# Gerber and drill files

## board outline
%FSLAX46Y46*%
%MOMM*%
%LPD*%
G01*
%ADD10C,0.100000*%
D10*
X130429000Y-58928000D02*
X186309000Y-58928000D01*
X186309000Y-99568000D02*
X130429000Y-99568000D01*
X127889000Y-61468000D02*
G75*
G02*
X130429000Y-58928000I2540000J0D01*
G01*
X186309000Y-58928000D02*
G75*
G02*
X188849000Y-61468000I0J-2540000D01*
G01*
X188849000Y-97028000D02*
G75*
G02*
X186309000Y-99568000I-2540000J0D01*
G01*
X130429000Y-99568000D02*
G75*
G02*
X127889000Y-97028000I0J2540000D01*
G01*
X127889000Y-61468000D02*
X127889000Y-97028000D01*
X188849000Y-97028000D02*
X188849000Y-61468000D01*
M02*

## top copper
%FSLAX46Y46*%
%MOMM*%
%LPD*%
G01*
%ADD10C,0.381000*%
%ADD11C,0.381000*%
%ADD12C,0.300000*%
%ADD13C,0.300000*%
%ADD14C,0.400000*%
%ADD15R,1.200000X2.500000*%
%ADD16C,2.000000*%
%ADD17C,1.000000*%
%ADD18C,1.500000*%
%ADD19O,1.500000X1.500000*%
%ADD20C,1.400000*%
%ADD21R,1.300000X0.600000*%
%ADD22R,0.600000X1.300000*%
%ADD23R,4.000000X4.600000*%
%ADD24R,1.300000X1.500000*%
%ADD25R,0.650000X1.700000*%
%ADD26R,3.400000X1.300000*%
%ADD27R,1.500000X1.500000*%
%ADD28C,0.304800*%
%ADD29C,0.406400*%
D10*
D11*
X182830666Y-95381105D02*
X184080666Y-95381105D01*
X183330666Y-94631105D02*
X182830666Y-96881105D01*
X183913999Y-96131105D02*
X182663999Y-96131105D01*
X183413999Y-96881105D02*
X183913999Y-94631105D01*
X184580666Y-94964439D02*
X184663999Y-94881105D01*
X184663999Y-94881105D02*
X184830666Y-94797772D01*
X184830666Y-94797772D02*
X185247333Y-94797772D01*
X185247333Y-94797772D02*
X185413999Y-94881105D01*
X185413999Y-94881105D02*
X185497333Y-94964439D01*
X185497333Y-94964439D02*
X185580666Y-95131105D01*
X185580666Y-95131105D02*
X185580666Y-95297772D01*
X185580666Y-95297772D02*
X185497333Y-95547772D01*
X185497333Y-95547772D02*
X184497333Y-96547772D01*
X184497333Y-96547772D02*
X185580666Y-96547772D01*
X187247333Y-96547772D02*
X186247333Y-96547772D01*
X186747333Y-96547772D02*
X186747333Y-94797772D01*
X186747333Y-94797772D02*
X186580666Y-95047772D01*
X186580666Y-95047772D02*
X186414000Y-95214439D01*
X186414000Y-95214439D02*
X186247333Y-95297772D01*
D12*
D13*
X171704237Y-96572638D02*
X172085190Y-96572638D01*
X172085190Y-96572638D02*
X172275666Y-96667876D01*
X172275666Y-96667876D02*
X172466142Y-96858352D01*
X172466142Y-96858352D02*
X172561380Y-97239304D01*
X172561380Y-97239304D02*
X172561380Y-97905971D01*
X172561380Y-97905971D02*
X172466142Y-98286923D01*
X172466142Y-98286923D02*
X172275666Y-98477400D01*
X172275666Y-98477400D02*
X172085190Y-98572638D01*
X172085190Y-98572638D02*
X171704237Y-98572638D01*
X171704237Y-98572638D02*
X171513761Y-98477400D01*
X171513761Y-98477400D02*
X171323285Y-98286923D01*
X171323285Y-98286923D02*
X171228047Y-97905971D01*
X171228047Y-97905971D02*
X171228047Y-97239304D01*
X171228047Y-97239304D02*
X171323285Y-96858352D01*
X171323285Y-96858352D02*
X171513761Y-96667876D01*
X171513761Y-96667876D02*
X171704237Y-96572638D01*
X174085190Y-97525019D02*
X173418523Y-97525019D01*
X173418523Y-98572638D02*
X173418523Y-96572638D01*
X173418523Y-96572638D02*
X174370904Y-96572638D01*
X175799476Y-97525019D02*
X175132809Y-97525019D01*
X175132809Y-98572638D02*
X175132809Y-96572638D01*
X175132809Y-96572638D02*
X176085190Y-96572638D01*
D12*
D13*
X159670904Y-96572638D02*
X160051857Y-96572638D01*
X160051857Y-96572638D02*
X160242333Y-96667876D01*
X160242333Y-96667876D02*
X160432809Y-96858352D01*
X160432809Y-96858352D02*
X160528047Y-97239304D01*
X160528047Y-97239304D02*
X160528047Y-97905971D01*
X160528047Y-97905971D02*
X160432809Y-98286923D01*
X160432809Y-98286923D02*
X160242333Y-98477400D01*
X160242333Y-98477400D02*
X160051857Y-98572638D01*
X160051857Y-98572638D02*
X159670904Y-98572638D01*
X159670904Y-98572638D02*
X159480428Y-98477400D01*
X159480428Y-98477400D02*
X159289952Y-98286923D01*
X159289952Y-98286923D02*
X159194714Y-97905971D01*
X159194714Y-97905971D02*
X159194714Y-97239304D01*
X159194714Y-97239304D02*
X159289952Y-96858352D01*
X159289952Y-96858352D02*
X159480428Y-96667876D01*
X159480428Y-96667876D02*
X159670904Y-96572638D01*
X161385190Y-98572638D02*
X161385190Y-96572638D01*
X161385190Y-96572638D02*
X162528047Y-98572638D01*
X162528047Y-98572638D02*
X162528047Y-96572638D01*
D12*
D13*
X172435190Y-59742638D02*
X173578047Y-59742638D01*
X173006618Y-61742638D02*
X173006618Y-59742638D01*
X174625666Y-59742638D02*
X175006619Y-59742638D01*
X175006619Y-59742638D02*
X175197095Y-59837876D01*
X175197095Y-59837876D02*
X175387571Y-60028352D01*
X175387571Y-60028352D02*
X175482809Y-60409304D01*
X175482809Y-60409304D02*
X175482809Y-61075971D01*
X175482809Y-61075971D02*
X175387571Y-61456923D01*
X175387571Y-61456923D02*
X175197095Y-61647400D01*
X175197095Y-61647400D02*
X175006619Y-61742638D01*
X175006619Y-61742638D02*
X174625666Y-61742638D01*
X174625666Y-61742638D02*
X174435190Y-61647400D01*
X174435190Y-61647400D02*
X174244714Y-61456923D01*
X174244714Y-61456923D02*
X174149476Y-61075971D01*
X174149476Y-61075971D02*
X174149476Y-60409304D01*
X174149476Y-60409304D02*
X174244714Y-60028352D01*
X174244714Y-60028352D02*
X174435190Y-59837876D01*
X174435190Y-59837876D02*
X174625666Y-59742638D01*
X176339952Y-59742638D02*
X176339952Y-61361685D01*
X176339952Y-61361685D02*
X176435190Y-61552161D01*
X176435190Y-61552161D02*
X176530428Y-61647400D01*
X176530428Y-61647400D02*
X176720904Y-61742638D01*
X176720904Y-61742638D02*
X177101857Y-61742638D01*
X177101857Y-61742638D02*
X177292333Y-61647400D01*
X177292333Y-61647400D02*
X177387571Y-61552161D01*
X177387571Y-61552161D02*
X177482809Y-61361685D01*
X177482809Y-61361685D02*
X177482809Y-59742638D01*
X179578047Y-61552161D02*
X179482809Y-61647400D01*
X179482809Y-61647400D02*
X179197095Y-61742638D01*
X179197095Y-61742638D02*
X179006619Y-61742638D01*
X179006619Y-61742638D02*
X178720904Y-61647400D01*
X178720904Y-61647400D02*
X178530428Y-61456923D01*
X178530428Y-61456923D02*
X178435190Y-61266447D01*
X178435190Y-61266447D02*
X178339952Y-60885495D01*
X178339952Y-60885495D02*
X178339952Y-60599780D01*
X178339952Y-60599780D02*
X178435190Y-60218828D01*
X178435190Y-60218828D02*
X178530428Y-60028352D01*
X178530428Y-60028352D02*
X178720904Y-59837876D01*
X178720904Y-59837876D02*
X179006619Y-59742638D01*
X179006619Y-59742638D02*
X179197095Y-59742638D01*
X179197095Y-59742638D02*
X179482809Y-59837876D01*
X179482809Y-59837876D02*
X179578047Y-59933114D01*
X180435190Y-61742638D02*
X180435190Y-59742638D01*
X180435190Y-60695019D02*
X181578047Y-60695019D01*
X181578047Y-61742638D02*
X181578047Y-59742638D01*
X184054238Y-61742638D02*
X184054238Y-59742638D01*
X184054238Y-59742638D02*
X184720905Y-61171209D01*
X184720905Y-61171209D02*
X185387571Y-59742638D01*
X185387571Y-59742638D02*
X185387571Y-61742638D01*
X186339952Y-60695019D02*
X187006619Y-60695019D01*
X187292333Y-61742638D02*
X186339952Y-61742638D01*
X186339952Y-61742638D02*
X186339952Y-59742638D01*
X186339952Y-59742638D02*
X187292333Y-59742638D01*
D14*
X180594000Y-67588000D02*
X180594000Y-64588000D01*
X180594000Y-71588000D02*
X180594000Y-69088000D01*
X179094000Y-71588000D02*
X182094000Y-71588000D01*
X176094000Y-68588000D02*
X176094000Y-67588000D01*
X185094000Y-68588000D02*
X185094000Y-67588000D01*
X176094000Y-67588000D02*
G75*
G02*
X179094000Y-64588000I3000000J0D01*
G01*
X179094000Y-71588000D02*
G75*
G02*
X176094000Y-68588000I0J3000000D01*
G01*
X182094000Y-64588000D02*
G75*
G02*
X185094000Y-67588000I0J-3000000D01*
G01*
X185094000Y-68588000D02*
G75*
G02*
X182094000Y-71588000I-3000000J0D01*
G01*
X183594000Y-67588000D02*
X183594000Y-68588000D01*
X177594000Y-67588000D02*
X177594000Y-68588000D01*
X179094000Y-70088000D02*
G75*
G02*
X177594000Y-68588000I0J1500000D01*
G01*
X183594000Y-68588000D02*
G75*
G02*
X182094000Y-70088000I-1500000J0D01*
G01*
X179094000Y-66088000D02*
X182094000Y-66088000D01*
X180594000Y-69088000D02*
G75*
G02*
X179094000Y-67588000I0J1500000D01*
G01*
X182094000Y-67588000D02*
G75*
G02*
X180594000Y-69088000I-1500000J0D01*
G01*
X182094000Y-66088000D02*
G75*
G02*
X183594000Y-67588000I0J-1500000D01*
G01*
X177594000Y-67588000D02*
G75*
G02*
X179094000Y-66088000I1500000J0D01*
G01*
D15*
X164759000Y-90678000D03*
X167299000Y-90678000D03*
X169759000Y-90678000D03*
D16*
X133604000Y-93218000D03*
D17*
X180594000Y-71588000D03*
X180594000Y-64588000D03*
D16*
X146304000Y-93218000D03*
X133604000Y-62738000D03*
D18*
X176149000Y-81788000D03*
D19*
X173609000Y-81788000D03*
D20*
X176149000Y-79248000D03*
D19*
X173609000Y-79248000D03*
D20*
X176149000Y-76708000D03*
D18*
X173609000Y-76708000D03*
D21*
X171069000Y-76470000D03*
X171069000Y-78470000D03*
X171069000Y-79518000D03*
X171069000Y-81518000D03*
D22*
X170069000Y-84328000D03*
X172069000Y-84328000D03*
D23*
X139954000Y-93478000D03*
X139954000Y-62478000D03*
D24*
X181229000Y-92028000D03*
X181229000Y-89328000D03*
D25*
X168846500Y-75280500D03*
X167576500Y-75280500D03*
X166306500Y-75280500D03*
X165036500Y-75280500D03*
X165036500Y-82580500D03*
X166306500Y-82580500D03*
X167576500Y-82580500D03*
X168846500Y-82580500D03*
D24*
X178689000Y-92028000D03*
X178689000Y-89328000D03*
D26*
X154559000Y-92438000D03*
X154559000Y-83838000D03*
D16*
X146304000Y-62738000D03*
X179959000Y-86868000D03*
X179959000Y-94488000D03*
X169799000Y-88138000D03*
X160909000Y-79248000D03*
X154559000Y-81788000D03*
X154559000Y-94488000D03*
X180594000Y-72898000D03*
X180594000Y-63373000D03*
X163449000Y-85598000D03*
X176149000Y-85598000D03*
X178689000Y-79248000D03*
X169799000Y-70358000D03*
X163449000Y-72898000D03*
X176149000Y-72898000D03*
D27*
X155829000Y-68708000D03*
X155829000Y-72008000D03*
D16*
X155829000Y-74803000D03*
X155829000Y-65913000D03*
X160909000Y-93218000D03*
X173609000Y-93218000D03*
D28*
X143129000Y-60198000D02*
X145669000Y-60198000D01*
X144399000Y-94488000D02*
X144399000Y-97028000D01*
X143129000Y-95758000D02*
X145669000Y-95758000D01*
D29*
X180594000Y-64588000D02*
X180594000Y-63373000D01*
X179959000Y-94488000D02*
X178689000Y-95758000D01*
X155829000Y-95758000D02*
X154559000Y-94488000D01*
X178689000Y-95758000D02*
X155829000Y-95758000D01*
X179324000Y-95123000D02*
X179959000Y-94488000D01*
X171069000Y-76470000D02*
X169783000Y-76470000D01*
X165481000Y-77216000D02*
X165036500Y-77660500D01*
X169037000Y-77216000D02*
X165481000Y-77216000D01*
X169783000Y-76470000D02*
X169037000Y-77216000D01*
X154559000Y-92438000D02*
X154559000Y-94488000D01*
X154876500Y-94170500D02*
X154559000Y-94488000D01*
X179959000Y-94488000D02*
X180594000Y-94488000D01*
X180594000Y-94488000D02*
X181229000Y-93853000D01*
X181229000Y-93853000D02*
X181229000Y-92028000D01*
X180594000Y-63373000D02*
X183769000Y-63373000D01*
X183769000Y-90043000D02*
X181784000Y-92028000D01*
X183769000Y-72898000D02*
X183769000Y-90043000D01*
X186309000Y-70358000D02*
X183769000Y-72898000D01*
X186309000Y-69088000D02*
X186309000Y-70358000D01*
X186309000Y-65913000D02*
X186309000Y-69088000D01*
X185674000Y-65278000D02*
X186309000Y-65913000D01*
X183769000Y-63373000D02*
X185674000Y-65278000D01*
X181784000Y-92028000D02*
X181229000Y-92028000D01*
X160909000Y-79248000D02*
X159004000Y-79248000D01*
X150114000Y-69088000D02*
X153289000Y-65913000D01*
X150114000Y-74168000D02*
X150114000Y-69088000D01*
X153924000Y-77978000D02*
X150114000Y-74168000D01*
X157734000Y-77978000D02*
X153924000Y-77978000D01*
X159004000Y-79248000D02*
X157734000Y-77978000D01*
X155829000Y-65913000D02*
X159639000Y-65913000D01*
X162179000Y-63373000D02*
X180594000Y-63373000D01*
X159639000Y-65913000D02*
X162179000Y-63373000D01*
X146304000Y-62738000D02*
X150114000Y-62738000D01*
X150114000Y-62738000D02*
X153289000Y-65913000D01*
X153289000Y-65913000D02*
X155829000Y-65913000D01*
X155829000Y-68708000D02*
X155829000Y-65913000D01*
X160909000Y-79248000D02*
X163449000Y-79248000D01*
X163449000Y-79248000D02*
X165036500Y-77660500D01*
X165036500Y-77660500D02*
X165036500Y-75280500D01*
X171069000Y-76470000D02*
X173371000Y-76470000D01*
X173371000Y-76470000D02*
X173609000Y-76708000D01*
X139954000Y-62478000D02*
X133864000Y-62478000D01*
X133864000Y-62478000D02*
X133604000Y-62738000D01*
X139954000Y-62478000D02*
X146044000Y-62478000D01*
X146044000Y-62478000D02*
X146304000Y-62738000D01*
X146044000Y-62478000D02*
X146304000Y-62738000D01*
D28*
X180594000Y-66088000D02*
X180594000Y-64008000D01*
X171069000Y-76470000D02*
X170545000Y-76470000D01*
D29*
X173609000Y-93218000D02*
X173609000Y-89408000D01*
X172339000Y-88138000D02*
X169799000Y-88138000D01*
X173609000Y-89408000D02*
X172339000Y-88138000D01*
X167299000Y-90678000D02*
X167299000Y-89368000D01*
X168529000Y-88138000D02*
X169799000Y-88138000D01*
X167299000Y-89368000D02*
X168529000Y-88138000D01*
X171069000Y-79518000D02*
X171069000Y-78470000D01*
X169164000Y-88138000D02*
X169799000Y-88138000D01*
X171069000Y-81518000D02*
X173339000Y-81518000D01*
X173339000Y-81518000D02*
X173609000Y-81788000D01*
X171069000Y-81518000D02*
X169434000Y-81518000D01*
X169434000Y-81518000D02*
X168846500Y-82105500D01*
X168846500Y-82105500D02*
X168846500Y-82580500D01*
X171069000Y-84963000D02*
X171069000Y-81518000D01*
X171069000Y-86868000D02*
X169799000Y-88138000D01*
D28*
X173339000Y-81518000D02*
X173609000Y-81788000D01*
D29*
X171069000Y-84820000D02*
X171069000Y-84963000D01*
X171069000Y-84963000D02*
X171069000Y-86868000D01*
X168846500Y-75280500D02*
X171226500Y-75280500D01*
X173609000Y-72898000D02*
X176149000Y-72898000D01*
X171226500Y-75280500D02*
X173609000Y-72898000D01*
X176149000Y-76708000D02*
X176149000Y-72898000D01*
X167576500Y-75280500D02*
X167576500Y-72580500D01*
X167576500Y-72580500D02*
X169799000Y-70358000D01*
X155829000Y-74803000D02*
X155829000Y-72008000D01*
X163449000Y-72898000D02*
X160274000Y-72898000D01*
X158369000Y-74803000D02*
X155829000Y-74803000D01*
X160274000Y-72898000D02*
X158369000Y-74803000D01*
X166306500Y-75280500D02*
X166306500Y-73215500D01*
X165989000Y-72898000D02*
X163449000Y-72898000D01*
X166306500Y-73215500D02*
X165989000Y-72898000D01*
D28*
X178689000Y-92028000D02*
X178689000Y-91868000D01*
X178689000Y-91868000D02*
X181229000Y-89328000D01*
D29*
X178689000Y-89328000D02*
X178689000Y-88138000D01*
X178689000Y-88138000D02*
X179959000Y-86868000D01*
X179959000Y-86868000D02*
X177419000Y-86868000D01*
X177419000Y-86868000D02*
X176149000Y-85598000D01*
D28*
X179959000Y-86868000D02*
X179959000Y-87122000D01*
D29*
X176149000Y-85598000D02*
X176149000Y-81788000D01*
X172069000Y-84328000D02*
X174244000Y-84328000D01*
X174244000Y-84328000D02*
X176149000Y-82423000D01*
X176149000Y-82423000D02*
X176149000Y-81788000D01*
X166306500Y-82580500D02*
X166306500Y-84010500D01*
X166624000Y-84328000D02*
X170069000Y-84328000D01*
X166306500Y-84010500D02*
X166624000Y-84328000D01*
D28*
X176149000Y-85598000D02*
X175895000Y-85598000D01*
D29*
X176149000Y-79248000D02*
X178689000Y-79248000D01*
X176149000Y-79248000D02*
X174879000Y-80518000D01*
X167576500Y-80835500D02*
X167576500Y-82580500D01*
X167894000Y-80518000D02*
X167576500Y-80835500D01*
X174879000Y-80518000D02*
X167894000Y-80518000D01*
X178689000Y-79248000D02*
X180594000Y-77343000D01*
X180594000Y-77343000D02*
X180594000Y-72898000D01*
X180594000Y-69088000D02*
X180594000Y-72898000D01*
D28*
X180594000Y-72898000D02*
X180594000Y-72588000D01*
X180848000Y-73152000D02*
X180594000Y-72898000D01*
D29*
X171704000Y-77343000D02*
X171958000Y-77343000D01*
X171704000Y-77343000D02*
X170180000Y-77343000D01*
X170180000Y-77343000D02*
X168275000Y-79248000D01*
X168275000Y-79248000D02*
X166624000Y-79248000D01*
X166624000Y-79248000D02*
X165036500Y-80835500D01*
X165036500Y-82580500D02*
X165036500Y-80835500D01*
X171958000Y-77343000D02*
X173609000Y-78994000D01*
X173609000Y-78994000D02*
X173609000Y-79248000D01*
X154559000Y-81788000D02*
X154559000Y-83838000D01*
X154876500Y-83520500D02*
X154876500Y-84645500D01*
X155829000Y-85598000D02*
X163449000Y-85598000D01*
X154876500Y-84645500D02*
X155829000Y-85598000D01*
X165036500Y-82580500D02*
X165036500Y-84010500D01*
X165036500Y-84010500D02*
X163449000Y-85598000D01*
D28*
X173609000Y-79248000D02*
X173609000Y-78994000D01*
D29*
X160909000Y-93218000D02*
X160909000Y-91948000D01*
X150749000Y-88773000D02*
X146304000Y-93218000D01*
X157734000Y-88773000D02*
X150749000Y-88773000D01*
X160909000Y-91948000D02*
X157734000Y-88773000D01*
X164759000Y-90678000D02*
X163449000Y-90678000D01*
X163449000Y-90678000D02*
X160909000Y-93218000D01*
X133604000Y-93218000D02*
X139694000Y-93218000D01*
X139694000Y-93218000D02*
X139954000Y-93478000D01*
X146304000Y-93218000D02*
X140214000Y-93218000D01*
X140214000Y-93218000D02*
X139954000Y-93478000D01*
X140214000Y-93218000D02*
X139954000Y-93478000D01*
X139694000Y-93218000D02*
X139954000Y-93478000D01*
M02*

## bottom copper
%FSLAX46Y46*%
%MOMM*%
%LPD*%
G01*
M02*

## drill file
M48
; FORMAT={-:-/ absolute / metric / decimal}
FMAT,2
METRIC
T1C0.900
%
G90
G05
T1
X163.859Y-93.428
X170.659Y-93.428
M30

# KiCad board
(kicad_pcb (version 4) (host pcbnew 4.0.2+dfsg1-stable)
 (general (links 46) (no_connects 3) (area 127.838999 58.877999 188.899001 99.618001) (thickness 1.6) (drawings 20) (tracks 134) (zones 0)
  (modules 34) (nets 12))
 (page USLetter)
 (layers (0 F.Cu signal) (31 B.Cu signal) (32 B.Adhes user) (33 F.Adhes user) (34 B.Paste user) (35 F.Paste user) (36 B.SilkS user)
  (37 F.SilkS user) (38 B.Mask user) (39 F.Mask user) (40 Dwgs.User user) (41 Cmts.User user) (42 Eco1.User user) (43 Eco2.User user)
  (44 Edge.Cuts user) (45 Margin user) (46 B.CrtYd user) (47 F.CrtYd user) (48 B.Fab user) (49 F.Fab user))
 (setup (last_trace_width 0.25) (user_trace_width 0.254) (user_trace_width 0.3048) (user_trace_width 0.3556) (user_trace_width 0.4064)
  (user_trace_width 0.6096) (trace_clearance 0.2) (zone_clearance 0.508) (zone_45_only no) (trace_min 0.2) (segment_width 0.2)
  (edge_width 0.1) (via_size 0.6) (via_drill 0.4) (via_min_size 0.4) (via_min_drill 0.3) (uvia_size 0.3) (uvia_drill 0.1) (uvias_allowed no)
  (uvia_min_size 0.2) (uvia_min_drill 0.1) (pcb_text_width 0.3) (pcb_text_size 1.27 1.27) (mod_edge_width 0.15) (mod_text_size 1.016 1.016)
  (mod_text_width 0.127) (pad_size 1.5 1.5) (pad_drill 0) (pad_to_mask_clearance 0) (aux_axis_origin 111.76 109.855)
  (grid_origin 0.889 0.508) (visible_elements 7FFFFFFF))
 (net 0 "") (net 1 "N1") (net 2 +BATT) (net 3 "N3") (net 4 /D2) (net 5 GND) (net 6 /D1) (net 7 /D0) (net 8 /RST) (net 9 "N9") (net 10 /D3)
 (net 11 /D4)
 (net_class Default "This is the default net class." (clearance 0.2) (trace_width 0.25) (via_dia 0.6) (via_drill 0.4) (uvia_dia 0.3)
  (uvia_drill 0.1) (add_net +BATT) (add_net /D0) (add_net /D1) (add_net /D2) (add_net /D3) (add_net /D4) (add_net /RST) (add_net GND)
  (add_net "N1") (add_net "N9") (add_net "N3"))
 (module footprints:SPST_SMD (layer F.Cu) (at 167.259 90.678)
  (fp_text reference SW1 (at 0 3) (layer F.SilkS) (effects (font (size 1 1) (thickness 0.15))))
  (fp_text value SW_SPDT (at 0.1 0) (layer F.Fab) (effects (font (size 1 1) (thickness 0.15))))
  (pad "" np_thru_hole circle (at 3.4 2.75) (size 0.9 0.9) (drill 0.9) (layers *.Cu *.Mask))
  (pad 1 smd rect (at -2.5 0) (size 1.2 2.5) (layers F.Cu F.Paste F.Mask) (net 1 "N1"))
  (pad 2 smd rect (at 0.04 0) (size 1.2 2.5) (layers F.Cu F.Paste F.Mask) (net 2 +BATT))
  (pad 3 smd rect (at 2.5 0) (size 1.2 2.5) (layers F.Cu F.Paste F.Mask) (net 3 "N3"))
  (pad "" np_thru_hole circle (at -3.4 2.75) (size 0.9 0.9) (drill 0.9) (layers *.Cu *.Mask)))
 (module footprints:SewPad (layer F.Cu) (at 133.604 93.218)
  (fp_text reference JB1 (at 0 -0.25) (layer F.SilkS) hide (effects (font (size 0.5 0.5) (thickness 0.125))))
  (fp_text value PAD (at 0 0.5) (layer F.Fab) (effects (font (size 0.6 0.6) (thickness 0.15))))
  (pad 1 smd circle (at 0 0) (size 2 2) (layers F.Cu F.Mask) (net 1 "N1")))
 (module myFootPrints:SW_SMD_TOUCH (layer F.Cu) (at 180.594 69.088)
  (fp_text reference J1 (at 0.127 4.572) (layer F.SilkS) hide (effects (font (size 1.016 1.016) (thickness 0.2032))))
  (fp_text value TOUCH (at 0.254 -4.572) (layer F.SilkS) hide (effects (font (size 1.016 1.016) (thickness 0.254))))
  (fp_line (start 0 -1.5) (end 0 -4.5) (layer F.Cu) (width 0.4)) (fp_line (start 0 2.5) (end 0 0) (layer F.Cu) (width 0.4))
  (fp_line (start -1.5 2.5) (end 1.5 2.5) (layer F.Cu) (width 0.4))
  (fp_line (start -4.5 -0.5) (end -4.5 -1.5) (layer F.Cu) (width 0.4))
  (fp_line (start 4.5 -0.5) (end 4.5 -1.5) (layer F.Cu) (width 0.4))
  (fp_arc (start -1.5 -1.5) (end -4.5 -1.5) (angle 90) (layer F.Cu) (width 0.4))
  (fp_arc (start -1.5 -0.5) (end -1.5 2.5) (angle 90) (layer F.Cu) (width 0.4))
  (fp_arc (start 1.5 -1.5) (end 1.5 -4.5) (angle 90) (layer F.Cu) (width 0.4))
  (fp_arc (start 1.5 -0.5) (end 4.5 -0.5) (angle 90) (layer F.Cu) (width 0.4))
  (fp_line (start 3 -1.5) (end 3 -0.5) (layer F.Cu) (width 0.4))
  (fp_line (start -3 -1.5) (end -3 -0.5) (layer F.Cu) (width 0.4))
  (fp_arc (start -1.5 -0.5) (end -1.5 1) (angle 90) (layer F.Cu) (width 0.4))
  (fp_arc (start 1.5 -0.5) (end 3 -0.5) (angle 90) (layer F.Cu) (width 0.4))
  (fp_line (start -1.5 -3) (end 1.5 -3) (layer F.Cu) (width 0.4))
  (fp_arc (start 0 -1.5) (end 0 0) (angle 90) (layer F.Cu) (width 0.4))
  (fp_arc (start 0 -1.5) (end 1.5 -1.5) (angle 90) (layer F.Cu) (width 0.4))
  (fp_arc (start 1.5 -1.5) (end 1.5 -3) (angle 90) (layer F.Cu) (width 0.4))
  (fp_arc (start -1.5 -1.5) (end -3 -1.5) (angle 90) (layer F.Cu) (width 0.4))
  (pad 2 smd circle (at 0 2.5) (size 1 1) (layers F.Cu) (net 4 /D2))
  (pad 1 smd circle (at 0 -4.5) (size 1 1) (layers F.Cu) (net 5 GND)))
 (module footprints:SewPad (layer F.Cu) (at 146.304 93.218)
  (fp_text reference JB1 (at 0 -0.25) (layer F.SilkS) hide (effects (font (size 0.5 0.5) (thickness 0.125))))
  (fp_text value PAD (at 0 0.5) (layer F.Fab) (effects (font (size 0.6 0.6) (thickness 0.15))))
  (pad 1 smd circle (at 0 0) (size 2 2) (layers F.Cu F.Mask) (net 1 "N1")))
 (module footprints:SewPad (layer F.Cu) (at 133.604 62.738)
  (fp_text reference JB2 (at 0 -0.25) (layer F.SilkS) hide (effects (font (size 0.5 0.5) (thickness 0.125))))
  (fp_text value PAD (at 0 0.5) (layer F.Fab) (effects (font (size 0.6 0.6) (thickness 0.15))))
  (pad 1 smd circle (at 0 0) (size 2 2) (layers F.Cu F.Mask) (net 5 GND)))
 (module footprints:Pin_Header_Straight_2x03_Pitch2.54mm (layer F.Cu) (at 176.149 81.788 180)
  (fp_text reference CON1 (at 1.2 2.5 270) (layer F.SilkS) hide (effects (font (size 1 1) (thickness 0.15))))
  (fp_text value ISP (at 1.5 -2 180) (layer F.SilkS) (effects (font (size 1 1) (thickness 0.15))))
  (pad 1 smd circle (at 0 0 180) (size 1.5 1.5) (layers F.Cu) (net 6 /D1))
  (pad 2 smd oval (at 2.54 0 180) (size 1.5 1.5) (layers F.Cu) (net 2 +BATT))
  (pad 3 smd circle (at 0 2.54 180) (size 1.4 1.4) (layers F.Cu) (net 4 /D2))
  (pad 4 smd oval (at 2.54 2.54 180) (size 1.5 1.5) (layers F.Cu) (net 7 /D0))
  (pad 5 smd circle (at 0 5.08 180) (size 1.4 1.4) (layers F.Cu) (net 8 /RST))
  (pad 6 smd circle (at 2.54 5.08 180) (size 1.5 1.5) (layers F.Cu) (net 5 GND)))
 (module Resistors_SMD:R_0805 (layer F.Cu) (at 171.069 77.47 270)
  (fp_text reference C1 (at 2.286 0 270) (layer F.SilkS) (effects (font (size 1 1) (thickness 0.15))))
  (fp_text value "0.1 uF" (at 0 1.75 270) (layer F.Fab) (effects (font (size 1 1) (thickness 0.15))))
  (pad 1 smd rect (at -1 0 270) (size 0.6 1.3) (layers F.Cu F.Paste F.Mask) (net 5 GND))
  (pad 2 smd rect (at 1 0 270) (size 0.6 1.3) (layers F.Cu F.Paste F.Mask) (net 2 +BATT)))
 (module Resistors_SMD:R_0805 (layer F.Cu) (at 171.069 80.518 270)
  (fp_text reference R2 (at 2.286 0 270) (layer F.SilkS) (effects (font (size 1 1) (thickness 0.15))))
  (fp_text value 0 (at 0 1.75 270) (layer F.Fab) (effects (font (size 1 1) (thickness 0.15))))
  (pad 1 smd rect (at -1 0 270) (size 0.6 1.3) (layers F.Cu F.Paste F.Mask) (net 2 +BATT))
  (pad 2 smd rect (at 1 0 270) (size 0.6 1.3) (layers F.Cu F.Paste F.Mask) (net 2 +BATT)))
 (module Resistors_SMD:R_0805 (layer F.Cu) (at 171.069 84.328)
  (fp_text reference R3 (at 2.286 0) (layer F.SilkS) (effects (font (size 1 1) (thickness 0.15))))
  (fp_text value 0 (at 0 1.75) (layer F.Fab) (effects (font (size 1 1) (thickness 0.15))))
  (pad 1 smd rect (at -1 0) (size 0.6 1.3) (layers F.Cu F.Paste F.Mask) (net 6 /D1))
  (pad 2 smd rect (at 1 0) (size 0.6 1.3) (layers F.Cu F.Paste F.Mask) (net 6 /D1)))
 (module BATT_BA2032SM (layer F.Cu) (at 139.954 77.978 90)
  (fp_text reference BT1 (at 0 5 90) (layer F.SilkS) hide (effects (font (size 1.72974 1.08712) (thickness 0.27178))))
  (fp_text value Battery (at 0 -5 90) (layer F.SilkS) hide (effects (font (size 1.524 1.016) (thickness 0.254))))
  (pad 1 smd rect (at -15.5 0 90) (size 4.6 4) (layers F.Cu F.Paste F.Mask) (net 1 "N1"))
  (pad 2 smd rect (at 15.5 0 90) (size 4.6 4) (layers F.Cu F.Paste F.Mask) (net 5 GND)))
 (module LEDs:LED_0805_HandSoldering (layer F.Cu) (at 181.229 90.678 90)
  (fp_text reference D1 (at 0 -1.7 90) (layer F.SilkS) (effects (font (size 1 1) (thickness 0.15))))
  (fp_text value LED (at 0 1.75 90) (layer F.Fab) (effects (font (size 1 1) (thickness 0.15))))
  (pad 1 smd rect (at -1.35 0 90) (size 1.5 1.3) (layers F.Cu F.Paste F.Mask) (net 5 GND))
  (pad 2 smd rect (at 1.35 0 90) (size 1.5 1.3) (layers F.Cu F.Paste F.Mask) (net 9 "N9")))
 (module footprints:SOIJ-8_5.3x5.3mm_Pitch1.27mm (layer F.Cu) (at 166.9415 78.9305 270)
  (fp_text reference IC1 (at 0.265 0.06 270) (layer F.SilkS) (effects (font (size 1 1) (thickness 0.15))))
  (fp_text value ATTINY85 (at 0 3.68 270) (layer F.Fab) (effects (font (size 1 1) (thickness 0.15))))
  (pad 1 smd rect (at -3.65 -1.905 270) (size 1.7 0.65) (layers F.Cu F.Paste F.Mask) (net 8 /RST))
  (pad 2 smd rect (at -3.65 -0.635 270) (size 1.7 0.65) (layers F.Cu F.Paste F.Mask) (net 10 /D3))
  (pad 3 smd rect (at -3.65 0.635 270) (size 1.7 0.65) (layers F.Cu F.Paste F.Mask) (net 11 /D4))
  (pad 4 smd rect (at -3.65 1.905 270) (size 1.7 0.65) (layers F.Cu F.Paste F.Mask) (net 5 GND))
  (pad 5 smd rect (at 3.65 1.905 270) (size 1.7 0.65) (layers F.Cu F.Paste F.Mask) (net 7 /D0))
  (pad 6 smd rect (at 3.65 0.635 270) (size 1.7 0.65) (layers F.Cu F.Paste F.Mask) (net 6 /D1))
  (pad 7 smd rect (at 3.65 -0.635 270) (size 1.7 0.65) (layers F.Cu F.Paste F.Mask) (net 4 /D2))
  (pad 8 smd rect (at 3.65 -1.905 270) (size 1.7 0.65) (layers F.Cu F.Paste F.Mask) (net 2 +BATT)))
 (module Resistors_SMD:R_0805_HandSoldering (layer F.Cu) (at 178.689 90.678 90)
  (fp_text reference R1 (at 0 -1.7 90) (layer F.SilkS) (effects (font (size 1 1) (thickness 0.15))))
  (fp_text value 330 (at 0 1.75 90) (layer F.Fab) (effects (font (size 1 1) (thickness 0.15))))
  (pad 1 smd rect (at -1.35 0 90) (size 1.5 1.3) (layers F.Cu F.Paste F.Mask) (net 9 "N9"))
  (pad 2 smd rect (at 1.35 0 90) (size 1.5 1.3) (layers F.Cu F.Paste F.Mask) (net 6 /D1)))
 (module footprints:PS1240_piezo (layer F.Cu) (at 154.559 88.138 90)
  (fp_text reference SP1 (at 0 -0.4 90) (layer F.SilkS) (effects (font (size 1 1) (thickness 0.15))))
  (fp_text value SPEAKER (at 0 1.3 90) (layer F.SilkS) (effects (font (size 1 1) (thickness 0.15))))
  (pad 1 smd rect (at -4.3 0 90) (size 1.3 3.4) (layers F.Cu F.Paste F.Mask) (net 5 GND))
  (pad 2 smd rect (at 4.3 0 90) (size 1.3 3.4) (layers F.Cu F.Paste F.Mask) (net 7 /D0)))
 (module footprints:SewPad (layer F.Cu) (at 146.304 62.738)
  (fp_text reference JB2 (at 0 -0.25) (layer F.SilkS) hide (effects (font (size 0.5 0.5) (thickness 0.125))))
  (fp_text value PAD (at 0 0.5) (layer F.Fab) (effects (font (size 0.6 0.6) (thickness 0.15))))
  (pad 1 smd circle (at 0 0) (size 2 2) (layers F.Cu F.Mask) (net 5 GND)))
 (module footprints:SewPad (layer F.Cu) (at 179.959 86.868 90)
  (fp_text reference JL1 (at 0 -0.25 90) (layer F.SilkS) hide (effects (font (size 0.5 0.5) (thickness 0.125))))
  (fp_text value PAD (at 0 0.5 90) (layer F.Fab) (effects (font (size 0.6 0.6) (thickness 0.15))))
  (pad 1 smd circle (at 0 0 90) (size 2 2) (layers F.Cu F.Mask) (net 6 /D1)))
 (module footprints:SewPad (layer F.Cu) (at 179.959 94.488 90)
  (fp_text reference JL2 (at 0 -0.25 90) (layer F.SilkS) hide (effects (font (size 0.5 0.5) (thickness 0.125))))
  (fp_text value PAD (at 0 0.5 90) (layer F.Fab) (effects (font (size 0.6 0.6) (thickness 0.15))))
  (pad 1 smd circle (at 0 0 90) (size 2 2) (layers F.Cu F.Mask) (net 5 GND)))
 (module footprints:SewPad (layer F.Cu) (at 169.799 88.138)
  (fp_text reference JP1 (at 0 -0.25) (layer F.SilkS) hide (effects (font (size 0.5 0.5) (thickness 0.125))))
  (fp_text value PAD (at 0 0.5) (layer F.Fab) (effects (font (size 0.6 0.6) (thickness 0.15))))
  (pad 1 smd circle (at 0 0) (size 2 2) (layers F.Cu F.Mask) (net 2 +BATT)))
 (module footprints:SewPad (layer F.Cu) (at 160.909 79.248)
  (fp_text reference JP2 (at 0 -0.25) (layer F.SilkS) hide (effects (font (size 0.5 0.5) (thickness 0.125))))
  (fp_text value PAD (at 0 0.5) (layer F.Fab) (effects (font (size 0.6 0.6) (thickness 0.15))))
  (pad 1 smd circle (at 0 0) (size 2 2) (layers F.Cu F.Mask) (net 5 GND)))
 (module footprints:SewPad (layer F.Cu) (at 154.559 81.788 180)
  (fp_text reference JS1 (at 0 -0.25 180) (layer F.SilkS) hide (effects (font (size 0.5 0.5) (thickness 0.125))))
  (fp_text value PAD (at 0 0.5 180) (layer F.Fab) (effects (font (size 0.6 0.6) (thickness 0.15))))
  (pad 1 smd circle (at 0 0 180) (size 2 2) (layers F.Cu F.Mask) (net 7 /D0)))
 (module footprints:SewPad (layer F.Cu) (at 154.559 94.488 180)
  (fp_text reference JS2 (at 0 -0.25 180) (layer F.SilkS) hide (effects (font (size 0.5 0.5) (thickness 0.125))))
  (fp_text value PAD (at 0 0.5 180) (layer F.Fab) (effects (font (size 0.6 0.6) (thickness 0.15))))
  (pad 1 smd circle (at 0 0 180) (size 2 2) (layers F.Cu F.Mask) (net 5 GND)))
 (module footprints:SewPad (layer F.Cu) (at 180.594 72.898 90)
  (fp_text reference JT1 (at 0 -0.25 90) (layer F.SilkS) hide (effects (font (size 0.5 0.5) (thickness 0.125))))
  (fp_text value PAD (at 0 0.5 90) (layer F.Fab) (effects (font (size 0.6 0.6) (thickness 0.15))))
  (pad 1 smd circle (at 0 0 90) (size 2 2) (layers F.Cu F.Mask) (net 4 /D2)))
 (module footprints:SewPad (layer F.Cu) (at 180.594 63.373 90)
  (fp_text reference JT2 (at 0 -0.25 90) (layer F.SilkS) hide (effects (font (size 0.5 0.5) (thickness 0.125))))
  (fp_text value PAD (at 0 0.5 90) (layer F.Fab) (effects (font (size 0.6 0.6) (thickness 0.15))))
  (pad 1 smd circle (at 0 0 90) (size 2 2) (layers F.Cu F.Mask) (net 5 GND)))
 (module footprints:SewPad (layer F.Cu) (at 163.449 85.598)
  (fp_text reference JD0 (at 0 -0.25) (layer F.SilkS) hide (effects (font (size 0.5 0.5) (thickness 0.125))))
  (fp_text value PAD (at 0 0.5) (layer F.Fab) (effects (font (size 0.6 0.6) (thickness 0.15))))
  (pad 1 smd circle (at 0 0) (size 2 2) (layers F.Cu F.Mask) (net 7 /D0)))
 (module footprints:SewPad (layer F.Cu) (at 176.149 85.598)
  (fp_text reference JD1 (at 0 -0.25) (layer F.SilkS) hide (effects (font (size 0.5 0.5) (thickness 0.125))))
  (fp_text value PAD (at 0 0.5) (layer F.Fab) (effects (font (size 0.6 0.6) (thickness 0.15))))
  (pad 1 smd circle (at 0 0) (size 2 2) (layers F.Cu F.Mask) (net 6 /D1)))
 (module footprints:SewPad (layer F.Cu) (at 178.689 79.248)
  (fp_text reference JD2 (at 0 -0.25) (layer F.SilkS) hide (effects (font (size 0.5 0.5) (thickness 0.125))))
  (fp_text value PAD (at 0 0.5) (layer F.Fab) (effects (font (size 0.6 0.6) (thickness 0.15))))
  (pad 1 smd circle (at 0 0) (size 2 2) (layers F.Cu F.Mask) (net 4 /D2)))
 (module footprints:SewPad (layer F.Cu) (at 169.799 70.358)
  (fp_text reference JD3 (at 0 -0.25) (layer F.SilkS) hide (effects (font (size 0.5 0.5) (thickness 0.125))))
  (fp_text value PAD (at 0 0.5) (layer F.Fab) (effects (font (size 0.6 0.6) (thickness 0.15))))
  (pad 1 smd circle (at 0 0) (size 2 2) (layers F.Cu F.Mask) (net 10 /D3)))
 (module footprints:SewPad (layer F.Cu) (at 163.449 72.898)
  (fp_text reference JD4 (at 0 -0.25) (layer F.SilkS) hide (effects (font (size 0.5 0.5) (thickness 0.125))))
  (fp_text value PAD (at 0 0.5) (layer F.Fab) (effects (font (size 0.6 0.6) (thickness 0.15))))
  (pad 1 smd circle (at 0 0) (size 2 2) (layers F.Cu F.Mask) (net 11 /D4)))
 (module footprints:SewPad (layer F.Cu) (at 176.149 72.898)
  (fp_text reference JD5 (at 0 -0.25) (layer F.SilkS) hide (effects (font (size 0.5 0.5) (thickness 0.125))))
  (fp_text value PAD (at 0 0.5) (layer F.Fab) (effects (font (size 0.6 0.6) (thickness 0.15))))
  (pad 1 smd circle (at 0 0) (size 2 2) (layers F.Cu F.Mask) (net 8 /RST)))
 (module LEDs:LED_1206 (layer F.Cu) (at 155.829 70.358 90)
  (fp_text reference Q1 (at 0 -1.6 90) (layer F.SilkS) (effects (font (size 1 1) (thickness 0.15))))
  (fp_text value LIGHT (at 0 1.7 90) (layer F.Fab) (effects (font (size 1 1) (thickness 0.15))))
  (pad 2 smd rect (at 1.65 0 270) (size 1.5 1.5) (layers F.Cu F.Paste F.Mask) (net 5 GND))
  (pad 1 smd rect (at -1.65 0 270) (size 1.5 1.5) (layers F.Cu F.Paste F.Mask) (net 11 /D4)))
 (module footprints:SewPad (layer F.Cu) (at 155.829 74.803)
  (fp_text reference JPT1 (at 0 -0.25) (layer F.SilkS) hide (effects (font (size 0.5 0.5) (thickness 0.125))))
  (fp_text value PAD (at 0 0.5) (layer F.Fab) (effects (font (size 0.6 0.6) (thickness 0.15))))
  (pad 1 smd circle (at 0 0) (size 2 2) (layers F.Cu F.Mask) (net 11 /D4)))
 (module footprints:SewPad (layer F.Cu) (at 155.829 65.913)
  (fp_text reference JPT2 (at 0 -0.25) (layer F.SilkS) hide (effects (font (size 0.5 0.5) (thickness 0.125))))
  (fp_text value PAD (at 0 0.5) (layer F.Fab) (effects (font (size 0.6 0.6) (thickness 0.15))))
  (pad 1 smd circle (at 0 0) (size 2 2) (layers F.Cu F.Mask) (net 5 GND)))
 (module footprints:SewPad (layer F.Cu) (at 160.909 93.218)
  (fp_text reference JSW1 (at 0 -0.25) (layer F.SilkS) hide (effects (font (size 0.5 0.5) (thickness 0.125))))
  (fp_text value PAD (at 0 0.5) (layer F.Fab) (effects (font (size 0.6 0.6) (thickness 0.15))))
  (pad 1 smd circle (at 0 0) (size 2 2) (layers F.Cu F.Mask) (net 1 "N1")))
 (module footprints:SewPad (layer F.Cu) (at 173.609 93.218)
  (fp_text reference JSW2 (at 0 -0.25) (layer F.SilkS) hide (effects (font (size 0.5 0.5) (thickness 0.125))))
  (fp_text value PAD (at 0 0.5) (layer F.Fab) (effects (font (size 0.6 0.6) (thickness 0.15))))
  (pad 1 smd circle (at 0 0) (size 2 2) (layers F.Cu F.Mask) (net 2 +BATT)))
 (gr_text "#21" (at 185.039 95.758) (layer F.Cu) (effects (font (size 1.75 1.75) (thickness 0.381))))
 (gr_line (start 130.429 58.928) (end 186.309 58.928) (angle 90) (layer Edge.Cuts) (width 0.1))
 (gr_line (start 186.309 99.568) (end 130.429 99.568) (angle 90) (layer Edge.Cuts) (width 0.1))
 (gr_arc (start 130.429 61.468) (end 127.889 61.468) (angle 90) (layer Edge.Cuts) (width 0.1))
 (gr_arc (start 186.309 61.468) (end 186.309 58.928) (angle 90) (layer Edge.Cuts) (width 0.1))
 (gr_arc (start 186.309 97.028) (end 188.849 97.028) (angle 90) (layer Edge.Cuts) (width 0.1))
 (gr_arc (start 130.429 97.028) (end 130.429 99.568) (angle 90) (layer Edge.Cuts) (width 0.1))
 (gr_line (start 127.889 61.468) (end 127.889 97.028) (angle 90) (layer Edge.Cuts) (width 0.1))
 (gr_line (start 188.849 97.028) (end 188.849 61.468) (angle 90) (layer Edge.Cuts) (width 0.1))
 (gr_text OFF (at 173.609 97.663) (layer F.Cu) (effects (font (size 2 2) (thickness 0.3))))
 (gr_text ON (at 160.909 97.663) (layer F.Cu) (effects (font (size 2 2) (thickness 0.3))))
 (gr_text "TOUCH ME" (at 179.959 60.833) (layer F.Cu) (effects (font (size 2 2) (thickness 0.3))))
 (segment (start 143.129 60.198) (end 145.669 60.198) (width 0.3048) (layer F.Cu) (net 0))
 (segment (start 144.399 94.488) (end 144.399 97.028) (width 0.3048) (layer F.Cu) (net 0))
 (segment (start 143.129 95.758) (end 145.669 95.758) (width 0.3048) (layer F.Cu) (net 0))
 (segment (start 180.594 64.588) (end 180.594 63.373) (width 0.4064) (layer F.Cu) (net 5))
 (segment (start 179.959 94.488) (end 178.689 95.758) (width 0.4064) (layer F.Cu) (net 5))
 (segment (start 155.829 95.758) (end 154.559 94.488) (width 0.4064) (layer F.Cu) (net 5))
 (segment (start 178.689 95.758) (end 155.829 95.758) (width 0.4064) (layer F.Cu) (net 5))
 (segment (start 179.324 95.123) (end 179.959 94.488) (width 0.4064) (layer F.Cu) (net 5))
 (segment (start 171.069 76.47) (end 169.783 76.47) (width 0.4064) (layer F.Cu) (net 5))
 (segment (start 165.481 77.216) (end 165.0365 77.6605) (width 0.4064) (layer F.Cu) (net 5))
 (segment (start 169.037 77.216) (end 165.481 77.216) (width 0.4064) (layer F.Cu) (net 5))
 (segment (start 169.783 76.47) (end 169.037 77.216) (width 0.4064) (layer F.Cu) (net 5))
 (segment (start 154.559 92.438) (end 154.559 94.488) (width 0.4064) (layer F.Cu) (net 5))
 (segment (start 154.8765 94.1705) (end 154.559 94.488) (width 0.4064) (layer F.Cu) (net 5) (status 30))
 (segment (start 179.959 94.488) (end 180.594 94.488) (width 0.4064) (layer F.Cu) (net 5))
 (segment (start 180.594 94.488) (end 181.229 93.853) (width 0.4064) (layer F.Cu) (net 5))
 (segment (start 181.229 93.853) (end 181.229 92.028) (width 0.4064) (layer F.Cu) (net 5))
 (segment (start 180.594 63.373) (end 183.769 63.373) (width 0.4064) (layer F.Cu) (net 5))
 (segment (start 183.769 90.043) (end 181.784 92.028) (width 0.4064) (layer F.Cu) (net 5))
 (segment (start 183.769 72.898) (end 183.769 90.043) (width 0.4064) (layer F.Cu) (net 5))
 (segment (start 186.309 70.358) (end 183.769 72.898) (width 0.4064) (layer F.Cu) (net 5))
 (segment (start 186.309 69.088) (end 186.309 70.358) (width 0.4064) (layer F.Cu) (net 5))
 (segment (start 186.309 65.913) (end 186.309 69.088) (width 0.4064) (layer F.Cu) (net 5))
 (segment (start 185.674 65.278) (end 186.309 65.913) (width 0.4064) (layer F.Cu) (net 5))
 (segment (start 183.769 63.373) (end 185.674 65.278) (width 0.4064) (layer F.Cu) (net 5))
 (segment (start 181.784 92.028) (end 181.229 92.028) (width 0.4064) (layer F.Cu) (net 5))
 (segment (start 160.909 79.248) (end 159.004 79.248) (width 0.4064) (layer F.Cu) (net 5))
 (segment (start 150.114 69.088) (end 153.289 65.913) (width 0.4064) (layer F.Cu) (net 5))
 (segment (start 150.114 74.168) (end 150.114 69.088) (width 0.4064) (layer F.Cu) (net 5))
 (segment (start 153.924 77.978) (end 150.114 74.168) (width 0.4064) (layer F.Cu) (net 5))
 (segment (start 157.734 77.978) (end 153.924 77.978) (width 0.4064) (layer F.Cu) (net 5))
 (segment (start 159.004 79.248) (end 157.734 77.978) (width 0.4064) (layer F.Cu) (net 5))
 (segment (start 155.829 65.913) (end 159.639 65.913) (width 0.4064) (layer F.Cu) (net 5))
 (segment (start 162.179 63.373) (end 180.594 63.373) (width 0.4064) (layer F.Cu) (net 5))
 (segment (start 159.639 65.913) (end 162.179 63.373) (width 0.4064) (layer F.Cu) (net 5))
 (segment (start 146.304 62.738) (end 150.114 62.738) (width 0.4064) (layer F.Cu) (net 5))
 (segment (start 150.114 62.738) (end 153.289 65.913) (width 0.4064) (layer F.Cu) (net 5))
 (segment (start 153.289 65.913) (end 155.829 65.913) (width 0.4064) (layer F.Cu) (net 5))
 (segment (start 155.829 68.708) (end 155.829 65.913) (width 0.4064) (layer F.Cu) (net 5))
 (segment (start 160.909 79.248) (end 163.449 79.248) (width 0.4064) (layer F.Cu) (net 5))
 (segment (start 163.449 79.248) (end 165.0365 77.6605) (width 0.4064) (layer F.Cu) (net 5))
 (segment (start 165.0365 77.6605) (end 165.0365 75.2805) (width 0.4064) (layer F.Cu) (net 5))
 (segment (start 171.069 76.47) (end 173.371 76.47) (width 0.4064) (layer F.Cu) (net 5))
 (segment (start 173.371 76.47) (end 173.609 76.708) (width 0.4064) (layer F.Cu) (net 5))
 (segment (start 139.954 62.478) (end 133.864 62.478) (width 0.4064) (layer F.Cu) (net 5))
 (segment (start 133.864 62.478) (end 133.604 62.738) (width 0.4064) (layer F.Cu) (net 5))
 (segment (start 139.954 62.478) (end 146.044 62.478) (width 0.4064) (layer F.Cu) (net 5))
 (segment (start 146.044 62.478) (end 146.304 62.738) (width 0.4064) (layer F.Cu) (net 5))
 (segment (start 146.044 62.478) (end 146.304 62.738) (width 0.4064) (layer F.Cu) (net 5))
 (segment (start 180.594 66.088) (end 180.594 64.008) (width 0.3048) (layer F.Cu) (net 5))
 (segment (start 171.069 76.47) (end 170.545 76.47) (width 0.3048) (layer F.Cu) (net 5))
 (segment (start 173.609 93.218) (end 173.609 89.408) (width 0.4064) (layer F.Cu) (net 2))
 (segment (start 172.339 88.138) (end 169.799 88.138) (width 0.4064) (layer F.Cu) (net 2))
 (segment (start 173.609 89.408) (end 172.339 88.138) (width 0.4064) (layer F.Cu) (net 2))
 (segment (start 167.299 90.678) (end 167.299 89.368) (width 0.4064) (layer F.Cu) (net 2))
 (segment (start 168.529 88.138) (end 169.799 88.138) (width 0.4064) (layer F.Cu) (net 2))
 (segment (start 167.299 89.368) (end 168.529 88.138) (width 0.4064) (layer F.Cu) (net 2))
 (segment (start 171.069 79.518) (end 171.069 78.47) (width 0.4064) (layer F.Cu) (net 2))
 (segment (start 169.164 88.138) (end 169.799 88.138) (width 0.4064) (layer F.Cu) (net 2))
 (segment (start 171.069 81.518) (end 173.339 81.518) (width 0.4064) (layer F.Cu) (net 2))
 (segment (start 173.339 81.518) (end 173.609 81.788) (width 0.4064) (layer F.Cu) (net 2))
 (segment (start 171.069 81.518) (end 169.434 81.518) (width 0.4064) (layer F.Cu) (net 2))
 (segment (start 169.434 81.518) (end 168.8465 82.1055) (width 0.4064) (layer F.Cu) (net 2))
 (segment (start 168.8465 82.1055) (end 168.8465 82.5805) (width 0.4064) (layer F.Cu) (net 2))
 (segment (start 171.069 84.963) (end 171.069 81.518) (width 0.4064) (layer F.Cu) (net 2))
 (segment (start 171.069 86.868) (end 169.799 88.138) (width 0.4064) (layer F.Cu) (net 2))
 (segment (start 173.339 81.518) (end 173.609 81.788) (width 0.3048) (layer F.Cu) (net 2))
 (segment (start 171.069 84.82) (end 171.069 84.963) (width 0.4064) (layer F.Cu) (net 2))
 (segment (start 171.069 84.963) (end 171.069 86.868) (width 0.4064) (layer F.Cu) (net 2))
 (segment (start 168.8465 75.2805) (end 171.2265 75.2805) (width 0.4064) (layer F.Cu) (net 8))
 (segment (start 173.609 72.898) (end 176.149 72.898) (width 0.4064) (layer F.Cu) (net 8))
 (segment (start 171.2265 75.2805) (end 173.609 72.898) (width 0.4064) (layer F.Cu) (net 8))
 (segment (start 176.149 76.708) (end 176.149 72.898) (width 0.4064) (layer F.Cu) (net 8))
 (segment (start 167.5765 75.2805) (end 167.5765 72.5805) (width 0.4064) (layer F.Cu) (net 10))
 (segment (start 167.5765 72.5805) (end 169.799 70.358) (width 0.4064) (layer F.Cu) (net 10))
 (segment (start 155.829 74.803) (end 155.829 72.008) (width 0.4064) (layer F.Cu) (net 11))
 (segment (start 163.449 72.898) (end 160.274 72.898) (width 0.4064) (layer F.Cu) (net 11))
 (segment (start 158.369 74.803) (end 155.829 74.803) (width 0.4064) (layer F.Cu) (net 11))
 (segment (start 160.274 72.898) (end 158.369 74.803) (width 0.4064) (layer F.Cu) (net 11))
 (segment (start 166.3065 75.2805) (end 166.3065 73.2155) (width 0.4064) (layer F.Cu) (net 11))
 (segment (start 165.989 72.898) (end 163.449 72.898) (width 0.4064) (layer F.Cu) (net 11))
 (segment (start 166.3065 73.2155) (end 165.989 72.898) (width 0.4064) (layer F.Cu) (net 11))
 (segment (start 178.689 92.028) (end 178.689 91.868) (width 0.3048) (layer F.Cu) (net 9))
 (segment (start 178.689 91.868) (end 181.229 89.328) (width 0.3048) (layer F.Cu) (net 9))
 (segment (start 178.689 89.328) (end 178.689 88.138) (width 0.4064) (layer F.Cu) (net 6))
 (segment (start 178.689 88.138) (end 179.959 86.868) (width 0.4064) (layer F.Cu) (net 6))
 (segment (start 179.959 86.868) (end 177.419 86.868) (width 0.4064) (layer F.Cu) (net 6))
 (segment (start 177.419 86.868) (end 176.149 85.598) (width 0.4064) (layer F.Cu) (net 6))
 (segment (start 179.959 86.868) (end 179.959 87.122) (width 0.3048) (layer F.Cu) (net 6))
 (segment (start 176.149 85.598) (end 176.149 81.788) (width 0.4064) (layer F.Cu) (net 6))
 (segment (start 172.069 84.328) (end 174.244 84.328) (width 0.4064) (layer F.Cu) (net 6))
 (segment (start 174.244 84.328) (end 176.149 82.423) (width 0.4064) (layer F.Cu) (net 6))
 (segment (start 176.149 82.423) (end 176.149 81.788) (width 0.4064) (layer F.Cu) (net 6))
 (segment (start 166.3065 82.5805) (end 166.3065 84.0105) (width 0.4064) (layer F.Cu) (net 6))
 (segment (start 166.624 84.328) (end 170.069 84.328) (width 0.4064) (layer F.Cu) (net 6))
 (segment (start 166.3065 84.0105) (end 166.624 84.328) (width 0.4064) (layer F.Cu) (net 6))
 (segment (start 176.149 85.598) (end 175.895 85.598) (width 0.3048) (layer F.Cu) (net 6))
 (segment (start 176.149 79.248) (end 178.689 79.248) (width 0.4064) (layer F.Cu) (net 4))
 (segment (start 176.149 79.248) (end 174.879 80.518) (width 0.4064) (layer F.Cu) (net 4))
 (segment (start 167.5765 80.8355) (end 167.5765 82.5805) (width 0.4064) (layer F.Cu) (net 4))
 (segment (start 167.894 80.518) (end 167.5765 80.8355) (width 0.4064) (layer F.Cu) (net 4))
 (segment (start 174.879 80.518) (end 167.894 80.518) (width 0.4064) (layer F.Cu) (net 4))
 (segment (start 178.689 79.248) (end 180.594 77.343) (width 0.4064) (layer F.Cu) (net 4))
 (segment (start 180.594 77.343) (end 180.594 72.898) (width 0.4064) (layer F.Cu) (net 4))
 (segment (start 180.594 69.088) (end 180.594 72.898) (width 0.4064) (layer F.Cu) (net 4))
 (segment (start 180.594 72.898) (end 180.594 72.588) (width 0.3048) (layer F.Cu) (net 4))
 (segment (start 180.848 73.152) (end 180.594 72.898) (width 0.3048) (layer F.Cu) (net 4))
 (segment (start 171.704 77.343) (end 171.958 77.343) (width 0.4064) (layer F.Cu) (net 7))
 (segment (start 171.704 77.343) (end 170.18 77.343) (width 0.4064) (layer F.Cu) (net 7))
 (segment (start 170.18 77.343) (end 168.275 79.248) (width 0.4064) (layer F.Cu) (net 7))
 (segment (start 168.275 79.248) (end 166.624 79.248) (width 0.4064) (layer F.Cu) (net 7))
 (segment (start 166.624 79.248) (end 165.0365 80.8355) (width 0.4064) (layer F.Cu) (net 7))
 (segment (start 165.0365 82.5805) (end 165.0365 80.8355) (width 0.4064) (layer F.Cu) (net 7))
 (segment (start 171.958 77.343) (end 173.609 78.994) (width 0.4064) (layer F.Cu) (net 7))
 (segment (start 173.609 78.994) (end 173.609 79.248) (width 0.4064) (layer F.Cu) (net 7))
 (segment (start 154.559 81.788) (end 154.559 83.838) (width 0.4064) (layer F.Cu) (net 7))
 (segment (start 154.8765 83.5205) (end 154.8765 84.6455) (width 0.4064) (layer F.Cu) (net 7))
 (segment (start 155.829 85.598) (end 163.449 85.598) (width 0.4064) (layer F.Cu) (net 7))
 (segment (start 154.8765 84.6455) (end 155.829 85.598) (width 0.4064) (layer F.Cu) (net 7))
 (segment (start 165.0365 82.5805) (end 165.0365 84.0105) (width 0.4064) (layer F.Cu) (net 7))
 (segment (start 165.0365 84.0105) (end 163.449 85.598) (width 0.4064) (layer F.Cu) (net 7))
 (segment (start 173.609 79.248) (end 173.609 78.994) (width 0.3048) (layer F.Cu) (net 7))
 (segment (start 160.909 93.218) (end 160.909 91.948) (width 0.4064) (layer F.Cu) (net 1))
 (segment (start 150.749 88.773) (end 146.304 93.218) (width 0.4064) (layer F.Cu) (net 1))
 (segment (start 157.734 88.773) (end 150.749 88.773) (width 0.4064) (layer F.Cu) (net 1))
 (segment (start 160.909 91.948) (end 157.734 88.773) (width 0.4064) (layer F.Cu) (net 1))
 (segment (start 164.759 90.678) (end 163.449 90.678) (width 0.4064) (layer F.Cu) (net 1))
 (segment (start 163.449 90.678) (end 160.909 93.218) (width 0.4064) (layer F.Cu) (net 1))
 (segment (start 133.604 93.218) (end 139.694 93.218) (width 0.4064) (layer F.Cu) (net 1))
 (segment (start 139.694 93.218) (end 139.954 93.478) (width 0.4064) (layer F.Cu) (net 1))
 (segment (start 146.304 93.218) (end 140.214 93.218) (width 0.4064) (layer F.Cu) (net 1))
 (segment (start 140.214 93.218) (end 139.954 93.478) (width 0.4064) (layer F.Cu) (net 1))
 (segment (start 140.214 93.218) (end 139.954 93.478) (width 0.4064) (layer F.Cu) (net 1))
 (segment (start 139.694 93.218) (end 139.954 93.478) (width 0.4064) (layer F.Cu) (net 1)))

